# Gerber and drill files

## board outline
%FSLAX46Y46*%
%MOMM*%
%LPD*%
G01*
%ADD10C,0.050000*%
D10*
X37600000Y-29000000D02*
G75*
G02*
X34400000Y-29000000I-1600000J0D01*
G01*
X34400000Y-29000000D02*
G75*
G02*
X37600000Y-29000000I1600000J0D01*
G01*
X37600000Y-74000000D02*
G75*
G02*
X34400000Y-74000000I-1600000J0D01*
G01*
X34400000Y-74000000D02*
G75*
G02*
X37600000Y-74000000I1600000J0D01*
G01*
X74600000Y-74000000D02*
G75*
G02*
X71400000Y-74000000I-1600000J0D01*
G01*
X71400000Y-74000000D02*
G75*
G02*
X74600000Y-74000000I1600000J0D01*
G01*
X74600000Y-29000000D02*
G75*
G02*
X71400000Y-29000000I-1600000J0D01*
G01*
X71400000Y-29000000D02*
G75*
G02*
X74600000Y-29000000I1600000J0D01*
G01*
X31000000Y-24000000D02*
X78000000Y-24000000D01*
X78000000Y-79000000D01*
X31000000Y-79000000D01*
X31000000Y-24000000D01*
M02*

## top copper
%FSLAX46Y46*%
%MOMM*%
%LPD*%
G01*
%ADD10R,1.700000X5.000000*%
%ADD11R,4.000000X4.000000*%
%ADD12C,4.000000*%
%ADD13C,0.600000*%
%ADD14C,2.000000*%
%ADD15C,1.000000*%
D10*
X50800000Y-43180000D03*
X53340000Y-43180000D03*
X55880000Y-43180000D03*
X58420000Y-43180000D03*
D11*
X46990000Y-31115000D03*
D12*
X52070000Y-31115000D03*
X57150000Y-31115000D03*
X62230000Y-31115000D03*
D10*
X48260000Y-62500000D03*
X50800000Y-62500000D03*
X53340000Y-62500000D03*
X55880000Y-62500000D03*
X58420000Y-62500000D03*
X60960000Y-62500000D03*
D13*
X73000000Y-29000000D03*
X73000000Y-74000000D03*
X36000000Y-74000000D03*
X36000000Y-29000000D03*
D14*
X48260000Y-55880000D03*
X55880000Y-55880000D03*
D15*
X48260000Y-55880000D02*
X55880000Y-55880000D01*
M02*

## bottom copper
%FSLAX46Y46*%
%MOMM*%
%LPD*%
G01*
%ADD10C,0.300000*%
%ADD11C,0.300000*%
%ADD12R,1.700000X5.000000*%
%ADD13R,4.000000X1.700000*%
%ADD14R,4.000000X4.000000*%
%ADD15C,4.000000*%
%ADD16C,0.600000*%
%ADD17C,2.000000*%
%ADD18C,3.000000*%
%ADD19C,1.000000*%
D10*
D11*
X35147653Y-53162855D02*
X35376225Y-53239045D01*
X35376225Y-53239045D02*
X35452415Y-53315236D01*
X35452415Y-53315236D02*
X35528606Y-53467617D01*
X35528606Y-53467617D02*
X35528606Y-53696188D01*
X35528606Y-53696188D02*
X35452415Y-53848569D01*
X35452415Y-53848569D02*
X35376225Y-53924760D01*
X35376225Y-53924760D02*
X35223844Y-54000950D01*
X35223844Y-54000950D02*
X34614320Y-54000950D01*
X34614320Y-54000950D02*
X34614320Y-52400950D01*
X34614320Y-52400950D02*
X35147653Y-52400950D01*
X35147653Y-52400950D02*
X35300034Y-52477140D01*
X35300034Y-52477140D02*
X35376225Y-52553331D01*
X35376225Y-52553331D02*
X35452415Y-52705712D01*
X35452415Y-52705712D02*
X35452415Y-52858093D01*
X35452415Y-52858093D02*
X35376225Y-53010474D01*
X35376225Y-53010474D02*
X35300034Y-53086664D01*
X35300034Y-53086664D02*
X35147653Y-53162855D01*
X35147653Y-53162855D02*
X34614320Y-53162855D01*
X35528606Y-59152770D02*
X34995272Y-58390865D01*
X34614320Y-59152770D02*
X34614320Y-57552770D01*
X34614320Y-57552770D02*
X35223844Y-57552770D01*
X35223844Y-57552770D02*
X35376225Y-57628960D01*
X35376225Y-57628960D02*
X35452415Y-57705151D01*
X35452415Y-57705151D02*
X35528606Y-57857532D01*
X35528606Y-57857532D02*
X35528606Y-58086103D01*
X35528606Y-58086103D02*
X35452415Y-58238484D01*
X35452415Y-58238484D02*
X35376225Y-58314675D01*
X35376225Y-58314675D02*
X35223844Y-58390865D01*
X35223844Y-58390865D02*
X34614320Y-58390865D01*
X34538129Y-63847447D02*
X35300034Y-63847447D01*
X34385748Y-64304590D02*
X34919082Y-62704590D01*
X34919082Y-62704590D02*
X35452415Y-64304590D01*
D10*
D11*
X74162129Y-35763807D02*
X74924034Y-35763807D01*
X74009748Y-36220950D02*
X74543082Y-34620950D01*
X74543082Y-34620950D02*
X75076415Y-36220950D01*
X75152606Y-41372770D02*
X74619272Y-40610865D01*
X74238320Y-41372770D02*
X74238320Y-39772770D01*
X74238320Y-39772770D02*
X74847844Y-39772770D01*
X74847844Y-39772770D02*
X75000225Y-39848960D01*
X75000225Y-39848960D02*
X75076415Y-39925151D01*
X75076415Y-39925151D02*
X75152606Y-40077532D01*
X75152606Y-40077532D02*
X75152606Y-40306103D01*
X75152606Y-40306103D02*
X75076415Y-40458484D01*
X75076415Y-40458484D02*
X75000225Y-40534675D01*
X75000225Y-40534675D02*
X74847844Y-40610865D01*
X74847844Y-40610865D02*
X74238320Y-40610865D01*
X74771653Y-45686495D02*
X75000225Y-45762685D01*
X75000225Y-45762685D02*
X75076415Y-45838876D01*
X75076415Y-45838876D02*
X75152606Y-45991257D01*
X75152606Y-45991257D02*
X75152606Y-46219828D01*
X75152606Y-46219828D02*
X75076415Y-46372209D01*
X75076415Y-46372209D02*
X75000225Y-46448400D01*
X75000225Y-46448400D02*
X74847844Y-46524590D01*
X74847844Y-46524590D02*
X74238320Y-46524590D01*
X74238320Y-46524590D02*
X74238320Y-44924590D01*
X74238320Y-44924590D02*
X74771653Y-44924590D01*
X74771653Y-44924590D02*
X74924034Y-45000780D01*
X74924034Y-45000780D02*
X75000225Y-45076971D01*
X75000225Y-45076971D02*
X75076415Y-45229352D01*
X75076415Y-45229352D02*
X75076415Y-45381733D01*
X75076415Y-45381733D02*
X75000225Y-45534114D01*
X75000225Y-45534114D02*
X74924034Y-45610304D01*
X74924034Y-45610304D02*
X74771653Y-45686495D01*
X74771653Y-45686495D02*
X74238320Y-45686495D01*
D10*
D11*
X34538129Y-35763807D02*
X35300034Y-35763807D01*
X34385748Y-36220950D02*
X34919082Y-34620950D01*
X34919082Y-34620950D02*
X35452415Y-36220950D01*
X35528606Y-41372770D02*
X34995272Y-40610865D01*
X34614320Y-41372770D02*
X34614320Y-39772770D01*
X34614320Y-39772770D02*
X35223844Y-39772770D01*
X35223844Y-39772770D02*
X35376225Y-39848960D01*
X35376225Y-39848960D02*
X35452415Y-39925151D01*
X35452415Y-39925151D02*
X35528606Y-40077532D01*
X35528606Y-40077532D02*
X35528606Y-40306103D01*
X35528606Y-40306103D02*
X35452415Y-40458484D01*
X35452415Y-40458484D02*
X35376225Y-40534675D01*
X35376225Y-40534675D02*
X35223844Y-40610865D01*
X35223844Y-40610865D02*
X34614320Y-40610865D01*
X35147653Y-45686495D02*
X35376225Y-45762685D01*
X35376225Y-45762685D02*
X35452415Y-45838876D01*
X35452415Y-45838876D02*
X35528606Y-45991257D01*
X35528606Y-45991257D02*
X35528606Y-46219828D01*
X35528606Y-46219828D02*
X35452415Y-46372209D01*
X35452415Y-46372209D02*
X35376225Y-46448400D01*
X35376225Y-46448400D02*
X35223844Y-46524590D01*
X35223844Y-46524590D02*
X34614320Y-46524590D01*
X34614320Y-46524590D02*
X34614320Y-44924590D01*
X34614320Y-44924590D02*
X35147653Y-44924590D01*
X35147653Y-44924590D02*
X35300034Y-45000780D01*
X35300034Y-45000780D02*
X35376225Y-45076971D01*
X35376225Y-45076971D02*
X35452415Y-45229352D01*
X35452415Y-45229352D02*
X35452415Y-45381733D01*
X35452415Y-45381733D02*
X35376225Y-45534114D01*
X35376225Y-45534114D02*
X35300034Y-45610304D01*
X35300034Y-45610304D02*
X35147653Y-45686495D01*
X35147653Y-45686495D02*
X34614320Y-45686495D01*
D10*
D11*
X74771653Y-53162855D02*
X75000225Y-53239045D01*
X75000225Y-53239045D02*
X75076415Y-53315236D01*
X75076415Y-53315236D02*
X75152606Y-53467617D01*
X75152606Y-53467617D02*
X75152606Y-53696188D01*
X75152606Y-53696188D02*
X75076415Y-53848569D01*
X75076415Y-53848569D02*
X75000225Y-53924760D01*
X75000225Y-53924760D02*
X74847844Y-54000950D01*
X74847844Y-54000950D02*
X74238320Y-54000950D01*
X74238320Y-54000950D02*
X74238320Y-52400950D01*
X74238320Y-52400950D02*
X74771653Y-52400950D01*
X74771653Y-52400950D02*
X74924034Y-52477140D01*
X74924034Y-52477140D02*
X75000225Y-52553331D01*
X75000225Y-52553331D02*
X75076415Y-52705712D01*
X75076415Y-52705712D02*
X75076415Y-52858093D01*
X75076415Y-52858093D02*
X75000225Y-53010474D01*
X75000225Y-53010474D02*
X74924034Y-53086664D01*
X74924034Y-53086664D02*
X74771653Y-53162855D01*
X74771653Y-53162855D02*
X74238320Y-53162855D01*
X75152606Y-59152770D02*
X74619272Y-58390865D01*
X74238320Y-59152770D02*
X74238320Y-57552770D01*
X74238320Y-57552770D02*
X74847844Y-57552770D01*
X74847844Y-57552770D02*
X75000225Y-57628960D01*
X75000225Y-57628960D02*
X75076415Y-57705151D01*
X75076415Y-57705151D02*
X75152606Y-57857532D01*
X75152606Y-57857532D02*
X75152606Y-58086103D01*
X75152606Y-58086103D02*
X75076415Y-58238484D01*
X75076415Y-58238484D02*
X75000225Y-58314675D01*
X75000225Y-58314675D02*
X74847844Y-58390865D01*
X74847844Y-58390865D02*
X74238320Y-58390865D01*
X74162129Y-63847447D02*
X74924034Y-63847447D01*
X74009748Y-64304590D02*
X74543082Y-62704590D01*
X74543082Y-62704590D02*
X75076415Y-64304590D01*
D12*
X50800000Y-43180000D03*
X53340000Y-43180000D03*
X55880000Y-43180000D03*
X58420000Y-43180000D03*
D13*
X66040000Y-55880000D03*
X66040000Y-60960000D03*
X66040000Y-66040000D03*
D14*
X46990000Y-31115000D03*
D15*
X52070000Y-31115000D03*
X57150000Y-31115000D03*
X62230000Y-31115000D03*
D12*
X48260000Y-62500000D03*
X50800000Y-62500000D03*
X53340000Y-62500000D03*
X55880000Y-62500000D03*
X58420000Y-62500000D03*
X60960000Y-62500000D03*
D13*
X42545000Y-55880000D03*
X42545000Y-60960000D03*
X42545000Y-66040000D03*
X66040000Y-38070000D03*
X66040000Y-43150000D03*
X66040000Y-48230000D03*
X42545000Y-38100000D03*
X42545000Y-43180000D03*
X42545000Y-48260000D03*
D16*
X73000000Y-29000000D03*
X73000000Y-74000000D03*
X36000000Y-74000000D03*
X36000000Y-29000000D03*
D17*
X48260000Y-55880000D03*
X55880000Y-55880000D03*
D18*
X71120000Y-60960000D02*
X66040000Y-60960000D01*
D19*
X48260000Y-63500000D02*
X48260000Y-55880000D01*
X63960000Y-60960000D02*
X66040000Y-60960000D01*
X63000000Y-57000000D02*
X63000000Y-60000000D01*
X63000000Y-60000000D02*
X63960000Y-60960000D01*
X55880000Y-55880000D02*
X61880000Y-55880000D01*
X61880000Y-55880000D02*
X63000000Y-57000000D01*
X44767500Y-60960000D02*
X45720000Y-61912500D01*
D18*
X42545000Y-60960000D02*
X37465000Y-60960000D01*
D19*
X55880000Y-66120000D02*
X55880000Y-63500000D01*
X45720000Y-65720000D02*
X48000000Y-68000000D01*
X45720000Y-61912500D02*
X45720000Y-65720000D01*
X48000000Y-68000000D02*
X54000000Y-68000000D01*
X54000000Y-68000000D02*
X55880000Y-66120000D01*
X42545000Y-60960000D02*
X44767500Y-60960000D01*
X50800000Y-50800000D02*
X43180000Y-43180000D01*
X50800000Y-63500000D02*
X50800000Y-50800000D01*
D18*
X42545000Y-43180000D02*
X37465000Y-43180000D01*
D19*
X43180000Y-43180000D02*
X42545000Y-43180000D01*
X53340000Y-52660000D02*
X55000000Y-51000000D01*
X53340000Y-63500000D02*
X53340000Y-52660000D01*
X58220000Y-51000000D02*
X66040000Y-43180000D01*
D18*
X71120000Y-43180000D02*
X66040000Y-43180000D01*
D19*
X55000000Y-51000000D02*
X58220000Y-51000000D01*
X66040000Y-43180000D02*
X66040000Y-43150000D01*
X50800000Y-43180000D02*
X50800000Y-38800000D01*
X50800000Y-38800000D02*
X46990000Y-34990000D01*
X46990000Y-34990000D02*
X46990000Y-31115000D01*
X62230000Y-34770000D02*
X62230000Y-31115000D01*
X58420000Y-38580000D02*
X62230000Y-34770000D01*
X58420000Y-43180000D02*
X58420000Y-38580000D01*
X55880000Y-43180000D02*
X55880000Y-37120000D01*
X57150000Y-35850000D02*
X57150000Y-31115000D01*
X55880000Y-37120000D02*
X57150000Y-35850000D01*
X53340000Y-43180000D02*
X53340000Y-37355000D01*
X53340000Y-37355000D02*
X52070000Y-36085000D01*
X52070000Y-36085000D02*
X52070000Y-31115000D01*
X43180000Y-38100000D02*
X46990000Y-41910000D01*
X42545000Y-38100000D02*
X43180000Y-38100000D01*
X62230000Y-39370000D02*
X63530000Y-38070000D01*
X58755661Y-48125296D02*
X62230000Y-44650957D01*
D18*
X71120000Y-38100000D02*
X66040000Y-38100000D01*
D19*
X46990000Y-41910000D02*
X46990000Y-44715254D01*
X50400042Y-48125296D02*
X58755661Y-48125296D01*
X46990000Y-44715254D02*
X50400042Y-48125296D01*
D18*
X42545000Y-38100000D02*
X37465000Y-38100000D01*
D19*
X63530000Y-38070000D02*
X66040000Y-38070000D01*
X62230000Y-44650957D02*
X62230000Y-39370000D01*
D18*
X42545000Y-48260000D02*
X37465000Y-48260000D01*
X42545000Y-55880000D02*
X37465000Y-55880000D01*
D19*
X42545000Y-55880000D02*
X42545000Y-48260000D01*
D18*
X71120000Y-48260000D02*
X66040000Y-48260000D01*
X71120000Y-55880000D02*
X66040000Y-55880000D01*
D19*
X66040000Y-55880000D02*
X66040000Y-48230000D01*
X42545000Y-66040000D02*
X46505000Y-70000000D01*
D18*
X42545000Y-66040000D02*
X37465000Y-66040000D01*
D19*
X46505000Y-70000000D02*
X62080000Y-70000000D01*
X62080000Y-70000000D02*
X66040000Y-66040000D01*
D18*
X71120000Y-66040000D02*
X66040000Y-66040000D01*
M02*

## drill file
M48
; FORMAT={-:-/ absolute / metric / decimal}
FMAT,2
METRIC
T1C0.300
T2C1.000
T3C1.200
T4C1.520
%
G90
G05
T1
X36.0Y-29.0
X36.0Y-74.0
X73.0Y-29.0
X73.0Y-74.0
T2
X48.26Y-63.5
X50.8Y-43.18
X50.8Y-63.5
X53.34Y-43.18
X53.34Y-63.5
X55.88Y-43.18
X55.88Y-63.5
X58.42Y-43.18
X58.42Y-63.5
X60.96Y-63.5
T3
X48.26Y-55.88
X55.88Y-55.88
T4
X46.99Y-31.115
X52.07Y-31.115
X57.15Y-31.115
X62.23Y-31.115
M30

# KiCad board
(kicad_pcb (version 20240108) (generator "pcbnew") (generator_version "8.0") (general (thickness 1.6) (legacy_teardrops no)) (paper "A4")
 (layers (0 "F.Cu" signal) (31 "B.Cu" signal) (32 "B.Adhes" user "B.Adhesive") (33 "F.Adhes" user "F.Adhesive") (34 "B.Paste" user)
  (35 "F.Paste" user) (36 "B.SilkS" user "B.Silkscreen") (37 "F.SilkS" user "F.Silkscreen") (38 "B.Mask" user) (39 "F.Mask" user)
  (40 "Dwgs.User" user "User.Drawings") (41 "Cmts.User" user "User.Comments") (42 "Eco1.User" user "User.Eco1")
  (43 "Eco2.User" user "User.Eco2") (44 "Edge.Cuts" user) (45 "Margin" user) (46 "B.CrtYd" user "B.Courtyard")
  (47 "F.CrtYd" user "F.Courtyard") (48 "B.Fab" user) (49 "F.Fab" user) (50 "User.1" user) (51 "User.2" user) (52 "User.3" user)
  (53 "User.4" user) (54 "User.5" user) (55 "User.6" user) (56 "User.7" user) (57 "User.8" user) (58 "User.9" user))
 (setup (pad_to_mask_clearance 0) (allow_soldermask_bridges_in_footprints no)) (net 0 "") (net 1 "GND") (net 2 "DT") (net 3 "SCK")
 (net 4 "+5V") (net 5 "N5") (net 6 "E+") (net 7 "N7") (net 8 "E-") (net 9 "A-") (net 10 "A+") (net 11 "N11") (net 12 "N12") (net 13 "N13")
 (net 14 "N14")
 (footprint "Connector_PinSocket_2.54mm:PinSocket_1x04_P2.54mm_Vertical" (layer "F.Cu") (at 50.8 43.18 90)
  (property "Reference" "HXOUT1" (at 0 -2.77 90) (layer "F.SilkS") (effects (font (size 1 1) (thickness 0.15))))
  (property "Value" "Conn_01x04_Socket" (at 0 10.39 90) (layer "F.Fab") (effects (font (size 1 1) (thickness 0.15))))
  (pad "1" thru_hole rect (at 0 0 90) (size 5 1.7) (drill 1) (layers "*.Cu" "*.Mask") (remove_unused_layers no) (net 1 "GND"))
  (pad "2" thru_hole rect (at 0 2.54 90) (size 5 1.7) (drill 1) (layers "*.Cu" "*.Mask") (remove_unused_layers no) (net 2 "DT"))
  (pad "3" thru_hole rect (at 0 5.08 90) (size 5 1.7) (drill 1) (layers "*.Cu" "*.Mask") (remove_unused_layers no) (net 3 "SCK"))
  (pad "4" thru_hole rect (at 0 7.62 90) (size 5 1.7) (drill 1) (layers "*.Cu" "*.Mask") (remove_unused_layers no) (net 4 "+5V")))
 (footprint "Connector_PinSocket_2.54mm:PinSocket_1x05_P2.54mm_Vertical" (layer "F.Cu") (at 66.04 55.88)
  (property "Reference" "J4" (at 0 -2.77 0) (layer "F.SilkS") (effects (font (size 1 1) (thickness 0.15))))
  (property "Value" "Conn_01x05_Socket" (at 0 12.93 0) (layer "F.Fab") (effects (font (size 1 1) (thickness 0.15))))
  (pad "1" smd rect (at 0 0) (size 4 1.7) (layers "B.Cu" "B.Paste" "B.Mask") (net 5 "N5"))
  (pad "3" smd rect (at 0 5.08) (size 4 1.7) (layers "B.Cu" "B.Paste" "B.Mask") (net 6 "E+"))
  (pad "5" smd rect (at 0 10.16) (size 4 1.7) (layers "B.Cu" "B.Paste" "B.Mask") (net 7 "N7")))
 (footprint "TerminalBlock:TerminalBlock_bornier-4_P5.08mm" (layer "F.Cu") (at 46.99 31.115)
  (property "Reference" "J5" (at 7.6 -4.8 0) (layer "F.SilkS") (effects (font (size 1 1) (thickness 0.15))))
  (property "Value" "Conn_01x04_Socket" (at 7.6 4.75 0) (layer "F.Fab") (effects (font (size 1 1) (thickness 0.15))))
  (pad "1" thru_hole rect (at 0 0) (size 4 4) (drill 1.52) (layers "*.Cu" "*.Mask") (remove_unused_layers no) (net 1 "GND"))
  (pad "2" thru_hole circle (at 5.08 0) (size 4 4) (drill 1.52) (layers "*.Cu" "*.Mask") (remove_unused_layers no) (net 2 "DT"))
  (pad "3" thru_hole circle (at 10.16 0) (size 4 4) (drill 1.52) (layers "*.Cu" "*.Mask") (remove_unused_layers no) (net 3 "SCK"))
  (pad "4" thru_hole circle (at 15.24 0) (size 4 4) (drill 1.52) (layers "*.Cu" "*.Mask") (remove_unused_layers no) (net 4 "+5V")))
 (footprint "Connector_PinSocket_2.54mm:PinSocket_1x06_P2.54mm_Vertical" (layer "F.Cu") (at 48.26 63.5 90)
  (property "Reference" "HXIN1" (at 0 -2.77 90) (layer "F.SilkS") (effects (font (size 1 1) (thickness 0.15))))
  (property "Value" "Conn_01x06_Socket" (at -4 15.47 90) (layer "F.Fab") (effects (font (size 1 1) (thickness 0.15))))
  (pad "1" thru_hole rect (at 0 0 90) (size 5 1.7) (drill 1 (offset 1 0)) (layers "*.Cu" "*.Mask") (remove_unused_layers no) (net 6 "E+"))
  (pad "2" thru_hole rect (at 0 2.54 90) (size 5 1.7) (drill 1 (offset 1 0)) (layers "*.Cu" "*.Mask") (remove_unused_layers no) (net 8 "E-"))
  (pad "3" thru_hole rect (at 0 5.08 90) (size 5 1.7) (drill 1 (offset 1 0)) (layers "*.Cu" "*.Mask") (remove_unused_layers no) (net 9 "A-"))
  (pad "4" thru_hole rect (at 0 7.62 90) (size 5 1.7) (drill 1 (offset 1 0)) (layers "*.Cu" "*.Mask") (remove_unused_layers no)
   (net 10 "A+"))
  (pad "5" thru_hole rect (at 0 10.16 90) (size 5 1.7) (drill 1 (offset 1 0)) (layers "*.Cu" "*.Mask") (remove_unused_layers no)
   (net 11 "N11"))
  (pad "6" thru_hole rect (at 0 12.7 90) (size 5 1.7) (drill 1 (offset 1 0)) (layers "*.Cu" "*.Mask") (remove_unused_layers no)
   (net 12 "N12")))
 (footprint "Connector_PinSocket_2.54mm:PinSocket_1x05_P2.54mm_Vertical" (layer "F.Cu") (at 42.545 55.88)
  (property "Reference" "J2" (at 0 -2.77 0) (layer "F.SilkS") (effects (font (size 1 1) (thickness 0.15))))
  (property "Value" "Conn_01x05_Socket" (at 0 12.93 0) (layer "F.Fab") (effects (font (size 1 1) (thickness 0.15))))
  (pad "1" smd rect (at 0 0) (size 4 1.7) (layers "B.Cu" "B.Paste" "B.Mask") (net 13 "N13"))
  (pad "3" smd rect (at 0 5.08) (size 4 1.7) (layers "B.Cu" "B.Paste" "B.Mask") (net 10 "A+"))
  (pad "5" smd rect (at 0 10.16) (size 4 1.7) (layers "B.Cu" "B.Paste" "B.Mask") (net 7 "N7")))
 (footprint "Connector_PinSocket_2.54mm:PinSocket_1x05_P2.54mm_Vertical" (layer "F.Cu") (at 66.04 38.07)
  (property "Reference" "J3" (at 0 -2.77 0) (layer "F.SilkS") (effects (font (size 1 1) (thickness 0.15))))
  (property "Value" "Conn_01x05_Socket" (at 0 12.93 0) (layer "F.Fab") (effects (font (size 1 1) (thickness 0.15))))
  (pad "1" smd rect (at 0 0) (size 4 1.7) (layers "B.Cu" "B.Paste" "B.Mask") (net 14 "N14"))
  (pad "3" smd rect (at 0 5.08) (size 4 1.7) (layers "B.Cu" "B.Paste" "B.Mask") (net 9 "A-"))
  (pad "5" smd rect (at 0 10.16) (size 4 1.7) (layers "B.Cu" "B.Paste" "B.Mask") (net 5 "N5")))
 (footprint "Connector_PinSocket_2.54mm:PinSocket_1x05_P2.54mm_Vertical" (layer "F.Cu") (at 42.545 38.1)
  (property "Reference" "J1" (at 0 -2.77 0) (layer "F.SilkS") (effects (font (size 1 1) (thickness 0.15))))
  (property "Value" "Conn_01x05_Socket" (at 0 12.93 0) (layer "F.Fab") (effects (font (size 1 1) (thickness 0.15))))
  (pad "1" smd rect (at 0 0) (size 4 1.7) (layers "B.Cu" "B.Paste" "B.Mask") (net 14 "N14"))
  (pad "3" smd rect (at 0 5.08) (size 4 1.7) (layers "B.Cu" "B.Paste" "B.Mask") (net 8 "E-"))
  (pad "5" smd rect (at 0 10.16) (size 4 1.7) (layers "B.Cu" "B.Paste" "B.Mask") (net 13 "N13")))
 (gr_circle (center 36 29) (end 37.6 29) (stroke (width 0.05) (type default)) (fill none) (layer "Edge.Cuts"))
 (gr_circle (center 36 74) (end 37.6 74) (stroke (width 0.05) (type default)) (fill none) (layer "Edge.Cuts"))
 (gr_circle (center 73 74) (end 74.6 74) (stroke (width 0.05) (type default)) (fill none) (layer "Edge.Cuts"))
 (gr_circle (center 73 29) (end 74.6 29) (stroke (width 0.05) (type default)) (fill none) (layer "Edge.Cuts"))
 (gr_rect (start 31 24) (end 78 79) (stroke (width 0.05) (type default)) (fill none) (layer "Edge.Cuts"))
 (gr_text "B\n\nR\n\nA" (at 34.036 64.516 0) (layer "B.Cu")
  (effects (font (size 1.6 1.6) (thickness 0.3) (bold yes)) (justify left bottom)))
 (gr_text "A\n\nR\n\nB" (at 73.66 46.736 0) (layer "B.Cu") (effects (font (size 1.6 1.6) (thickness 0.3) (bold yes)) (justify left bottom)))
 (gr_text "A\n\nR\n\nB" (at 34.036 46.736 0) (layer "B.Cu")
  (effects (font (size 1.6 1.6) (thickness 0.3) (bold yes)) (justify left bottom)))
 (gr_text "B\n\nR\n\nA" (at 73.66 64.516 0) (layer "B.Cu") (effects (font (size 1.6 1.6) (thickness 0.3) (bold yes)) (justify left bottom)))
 (via (at 73 29) (size 0.6) (drill 0.3) (layers "F.Cu" "B.Cu") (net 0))
 (via (at 73 74) (size 0.6) (drill 0.3) (layers "F.Cu" "B.Cu") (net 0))
 (via (at 36 74) (size 0.6) (drill 0.3) (layers "F.Cu" "B.Cu") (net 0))
 (via (at 36 29) (size 0.6) (drill 0.3) (layers "F.Cu" "B.Cu") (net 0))
 (segment (start 48.26 55.88) (end 55.88 55.88) (width 1) (layer "F.Cu") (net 6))
 (via (at 48.26 55.88) (size 2) (drill 1.2) (layers "F.Cu" "B.Cu") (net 6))
 (via (at 55.88 55.88) (size 2) (drill 1.2) (layers "F.Cu" "B.Cu") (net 6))
 (segment (start 71.12 60.96) (end 66.04 60.96) (width 3) (layer "B.Cu") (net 6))
 (segment (start 48.26 63.5) (end 48.26 55.88) (width 1) (layer "B.Cu") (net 6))
 (segment (start 63.96 60.96) (end 66.04 60.96) (width 1) (layer "B.Cu") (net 6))
 (segment (start 63 57) (end 63 60) (width 1) (layer "B.Cu") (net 6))
 (segment (start 63 60) (end 63.96 60.96) (width 1) (layer "B.Cu") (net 6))
 (segment (start 55.88 55.88) (end 61.88 55.88) (width 1) (layer "B.Cu") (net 6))
 (segment (start 61.88 55.88) (end 63 57) (width 1) (layer "B.Cu") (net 6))
 (segment (start 44.7675 60.96) (end 45.72 61.9125) (width 1) (layer "B.Cu") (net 10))
 (segment (start 42.545 60.96) (end 37.465 60.96) (width 3) (layer "B.Cu") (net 10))
 (segment (start 55.88 66.12) (end 55.88 63.5) (width 1) (layer "B.Cu") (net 10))
 (segment (start 45.72 65.72) (end 48 68) (width 1) (layer "B.Cu") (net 10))
 (segment (start 45.72 61.9125) (end 45.72 65.72) (width 1) (layer "B.Cu") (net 10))
 (segment (start 48 68) (end 54 68) (width 1) (layer "B.Cu") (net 10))
 (segment (start 54 68) (end 55.88 66.12) (width 1) (layer "B.Cu") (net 10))
 (segment (start 42.545 60.96) (end 44.7675 60.96) (width 1) (layer "B.Cu") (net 10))
 (segment (start 50.8 50.8) (end 43.18 43.18) (width 1) (layer "B.Cu") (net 8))
 (segment (start 50.8 63.5) (end 50.8 50.8) (width 1) (layer "B.Cu") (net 8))
 (segment (start 42.545 43.18) (end 37.465 43.18) (width 3) (layer "B.Cu") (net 8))
 (segment (start 43.18 43.18) (end 42.545 43.18) (width 1) (layer "B.Cu") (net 8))
 (segment (start 53.34 52.66) (end 55 51) (width 1) (layer "B.Cu") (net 9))
 (segment (start 53.34 63.5) (end 53.34 52.66) (width 1) (layer "B.Cu") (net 9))
 (segment (start 58.22 51) (end 66.04 43.18) (width 1) (layer "B.Cu") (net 9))
 (segment (start 71.12 43.18) (end 66.04 43.18) (width 3) (layer "B.Cu") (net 9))
 (segment (start 55 51) (end 58.22 51) (width 1) (layer "B.Cu") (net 9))
 (segment (start 66.04 43.18) (end 66.04 43.15) (width 1) (layer "B.Cu") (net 9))
 (segment (start 50.8 43.18) (end 50.8 38.8) (width 1) (layer "B.Cu") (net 1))
 (segment (start 50.8 38.8) (end 46.99 34.99) (width 1) (layer "B.Cu") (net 1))
 (segment (start 46.99 34.99) (end 46.99 31.115) (width 1) (layer "B.Cu") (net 1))
 (segment (start 62.23 34.77) (end 62.23 31.115) (width 1) (layer "B.Cu") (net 4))
 (segment (start 58.42 38.58) (end 62.23 34.77) (width 1) (layer "B.Cu") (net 4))
 (segment (start 58.42 43.18) (end 58.42 38.58) (width 1) (layer "B.Cu") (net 4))
 (segment (start 55.88 43.18) (end 55.88 37.12) (width 1) (layer "B.Cu") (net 3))
 (segment (start 57.15 35.85) (end 57.15 31.115) (width 1) (layer "B.Cu") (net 3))
 (segment (start 55.88 37.12) (end 57.15 35.85) (width 1) (layer "B.Cu") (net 3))
 (segment (start 53.34 43.18) (end 53.34 37.355) (width 1) (layer "B.Cu") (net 2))
 (segment (start 53.34 37.355) (end 52.07 36.085) (width 1) (layer "B.Cu") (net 2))
 (segment (start 52.07 36.085) (end 52.07 31.115) (width 1) (layer "B.Cu") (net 2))
 (segment (start 43.18 38.1) (end 46.99 41.91) (width 1) (layer "B.Cu") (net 14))
 (segment (start 42.545 38.1) (end 43.18 38.1) (width 1) (layer "B.Cu") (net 14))
 (segment (start 62.23 39.37) (end 63.53 38.07) (width 1) (layer "B.Cu") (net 14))
 (segment (start 58.755661 48.125296) (end 62.23 44.650957) (width 1) (layer "B.Cu") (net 14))
 (segment (start 71.12 38.1) (end 66.04 38.1) (width 3) (layer "B.Cu") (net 14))
 (segment (start 46.99 41.91) (end 46.99 44.715254) (width 1) (layer "B.Cu") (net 14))
 (segment (start 50.400042 48.125296) (end 58.755661 48.125296) (width 1) (layer "B.Cu") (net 14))
 (segment (start 46.99 44.715254) (end 50.400042 48.125296) (width 1) (layer "B.Cu") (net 14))
 (segment (start 42.545 38.1) (end 37.465 38.1) (width 3) (layer "B.Cu") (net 14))
 (segment (start 63.53 38.07) (end 66.04 38.07) (width 1) (layer "B.Cu") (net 14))
 (segment (start 62.23 44.650957) (end 62.23 39.37) (width 1) (layer "B.Cu") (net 14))
 (segment (start 42.545 48.26) (end 37.465 48.26) (width 3) (layer "B.Cu") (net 13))
 (segment (start 42.545 55.88) (end 37.465 55.88) (width 3) (layer "B.Cu") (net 13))
 (segment (start 42.545 55.88) (end 42.545 48.26) (width 1) (layer "B.Cu") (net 13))
 (segment (start 71.12 48.26) (end 66.04 48.26) (width 3) (layer "B.Cu") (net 5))
 (segment (start 71.12 55.88) (end 66.04 55.88) (width 3) (layer "B.Cu") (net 5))
 (segment (start 66.04 55.88) (end 66.04 48.23) (width 1) (layer "B.Cu") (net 5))
 (segment (start 42.545 66.04) (end 46.505 70) (width 1) (layer "B.Cu") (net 7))
 (segment (start 42.545 66.04) (end 37.465 66.04) (width 3) (layer "B.Cu") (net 7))
 (segment (start 46.505 70) (end 62.08 70) (width 1) (layer "B.Cu") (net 7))
 (segment (start 62.08 70) (end 66.04 66.04) (width 1) (layer "B.Cu") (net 7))
 (segment (start 71.12 66.04) (end 66.04 66.04) (width 3) (layer "B.Cu") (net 7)))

